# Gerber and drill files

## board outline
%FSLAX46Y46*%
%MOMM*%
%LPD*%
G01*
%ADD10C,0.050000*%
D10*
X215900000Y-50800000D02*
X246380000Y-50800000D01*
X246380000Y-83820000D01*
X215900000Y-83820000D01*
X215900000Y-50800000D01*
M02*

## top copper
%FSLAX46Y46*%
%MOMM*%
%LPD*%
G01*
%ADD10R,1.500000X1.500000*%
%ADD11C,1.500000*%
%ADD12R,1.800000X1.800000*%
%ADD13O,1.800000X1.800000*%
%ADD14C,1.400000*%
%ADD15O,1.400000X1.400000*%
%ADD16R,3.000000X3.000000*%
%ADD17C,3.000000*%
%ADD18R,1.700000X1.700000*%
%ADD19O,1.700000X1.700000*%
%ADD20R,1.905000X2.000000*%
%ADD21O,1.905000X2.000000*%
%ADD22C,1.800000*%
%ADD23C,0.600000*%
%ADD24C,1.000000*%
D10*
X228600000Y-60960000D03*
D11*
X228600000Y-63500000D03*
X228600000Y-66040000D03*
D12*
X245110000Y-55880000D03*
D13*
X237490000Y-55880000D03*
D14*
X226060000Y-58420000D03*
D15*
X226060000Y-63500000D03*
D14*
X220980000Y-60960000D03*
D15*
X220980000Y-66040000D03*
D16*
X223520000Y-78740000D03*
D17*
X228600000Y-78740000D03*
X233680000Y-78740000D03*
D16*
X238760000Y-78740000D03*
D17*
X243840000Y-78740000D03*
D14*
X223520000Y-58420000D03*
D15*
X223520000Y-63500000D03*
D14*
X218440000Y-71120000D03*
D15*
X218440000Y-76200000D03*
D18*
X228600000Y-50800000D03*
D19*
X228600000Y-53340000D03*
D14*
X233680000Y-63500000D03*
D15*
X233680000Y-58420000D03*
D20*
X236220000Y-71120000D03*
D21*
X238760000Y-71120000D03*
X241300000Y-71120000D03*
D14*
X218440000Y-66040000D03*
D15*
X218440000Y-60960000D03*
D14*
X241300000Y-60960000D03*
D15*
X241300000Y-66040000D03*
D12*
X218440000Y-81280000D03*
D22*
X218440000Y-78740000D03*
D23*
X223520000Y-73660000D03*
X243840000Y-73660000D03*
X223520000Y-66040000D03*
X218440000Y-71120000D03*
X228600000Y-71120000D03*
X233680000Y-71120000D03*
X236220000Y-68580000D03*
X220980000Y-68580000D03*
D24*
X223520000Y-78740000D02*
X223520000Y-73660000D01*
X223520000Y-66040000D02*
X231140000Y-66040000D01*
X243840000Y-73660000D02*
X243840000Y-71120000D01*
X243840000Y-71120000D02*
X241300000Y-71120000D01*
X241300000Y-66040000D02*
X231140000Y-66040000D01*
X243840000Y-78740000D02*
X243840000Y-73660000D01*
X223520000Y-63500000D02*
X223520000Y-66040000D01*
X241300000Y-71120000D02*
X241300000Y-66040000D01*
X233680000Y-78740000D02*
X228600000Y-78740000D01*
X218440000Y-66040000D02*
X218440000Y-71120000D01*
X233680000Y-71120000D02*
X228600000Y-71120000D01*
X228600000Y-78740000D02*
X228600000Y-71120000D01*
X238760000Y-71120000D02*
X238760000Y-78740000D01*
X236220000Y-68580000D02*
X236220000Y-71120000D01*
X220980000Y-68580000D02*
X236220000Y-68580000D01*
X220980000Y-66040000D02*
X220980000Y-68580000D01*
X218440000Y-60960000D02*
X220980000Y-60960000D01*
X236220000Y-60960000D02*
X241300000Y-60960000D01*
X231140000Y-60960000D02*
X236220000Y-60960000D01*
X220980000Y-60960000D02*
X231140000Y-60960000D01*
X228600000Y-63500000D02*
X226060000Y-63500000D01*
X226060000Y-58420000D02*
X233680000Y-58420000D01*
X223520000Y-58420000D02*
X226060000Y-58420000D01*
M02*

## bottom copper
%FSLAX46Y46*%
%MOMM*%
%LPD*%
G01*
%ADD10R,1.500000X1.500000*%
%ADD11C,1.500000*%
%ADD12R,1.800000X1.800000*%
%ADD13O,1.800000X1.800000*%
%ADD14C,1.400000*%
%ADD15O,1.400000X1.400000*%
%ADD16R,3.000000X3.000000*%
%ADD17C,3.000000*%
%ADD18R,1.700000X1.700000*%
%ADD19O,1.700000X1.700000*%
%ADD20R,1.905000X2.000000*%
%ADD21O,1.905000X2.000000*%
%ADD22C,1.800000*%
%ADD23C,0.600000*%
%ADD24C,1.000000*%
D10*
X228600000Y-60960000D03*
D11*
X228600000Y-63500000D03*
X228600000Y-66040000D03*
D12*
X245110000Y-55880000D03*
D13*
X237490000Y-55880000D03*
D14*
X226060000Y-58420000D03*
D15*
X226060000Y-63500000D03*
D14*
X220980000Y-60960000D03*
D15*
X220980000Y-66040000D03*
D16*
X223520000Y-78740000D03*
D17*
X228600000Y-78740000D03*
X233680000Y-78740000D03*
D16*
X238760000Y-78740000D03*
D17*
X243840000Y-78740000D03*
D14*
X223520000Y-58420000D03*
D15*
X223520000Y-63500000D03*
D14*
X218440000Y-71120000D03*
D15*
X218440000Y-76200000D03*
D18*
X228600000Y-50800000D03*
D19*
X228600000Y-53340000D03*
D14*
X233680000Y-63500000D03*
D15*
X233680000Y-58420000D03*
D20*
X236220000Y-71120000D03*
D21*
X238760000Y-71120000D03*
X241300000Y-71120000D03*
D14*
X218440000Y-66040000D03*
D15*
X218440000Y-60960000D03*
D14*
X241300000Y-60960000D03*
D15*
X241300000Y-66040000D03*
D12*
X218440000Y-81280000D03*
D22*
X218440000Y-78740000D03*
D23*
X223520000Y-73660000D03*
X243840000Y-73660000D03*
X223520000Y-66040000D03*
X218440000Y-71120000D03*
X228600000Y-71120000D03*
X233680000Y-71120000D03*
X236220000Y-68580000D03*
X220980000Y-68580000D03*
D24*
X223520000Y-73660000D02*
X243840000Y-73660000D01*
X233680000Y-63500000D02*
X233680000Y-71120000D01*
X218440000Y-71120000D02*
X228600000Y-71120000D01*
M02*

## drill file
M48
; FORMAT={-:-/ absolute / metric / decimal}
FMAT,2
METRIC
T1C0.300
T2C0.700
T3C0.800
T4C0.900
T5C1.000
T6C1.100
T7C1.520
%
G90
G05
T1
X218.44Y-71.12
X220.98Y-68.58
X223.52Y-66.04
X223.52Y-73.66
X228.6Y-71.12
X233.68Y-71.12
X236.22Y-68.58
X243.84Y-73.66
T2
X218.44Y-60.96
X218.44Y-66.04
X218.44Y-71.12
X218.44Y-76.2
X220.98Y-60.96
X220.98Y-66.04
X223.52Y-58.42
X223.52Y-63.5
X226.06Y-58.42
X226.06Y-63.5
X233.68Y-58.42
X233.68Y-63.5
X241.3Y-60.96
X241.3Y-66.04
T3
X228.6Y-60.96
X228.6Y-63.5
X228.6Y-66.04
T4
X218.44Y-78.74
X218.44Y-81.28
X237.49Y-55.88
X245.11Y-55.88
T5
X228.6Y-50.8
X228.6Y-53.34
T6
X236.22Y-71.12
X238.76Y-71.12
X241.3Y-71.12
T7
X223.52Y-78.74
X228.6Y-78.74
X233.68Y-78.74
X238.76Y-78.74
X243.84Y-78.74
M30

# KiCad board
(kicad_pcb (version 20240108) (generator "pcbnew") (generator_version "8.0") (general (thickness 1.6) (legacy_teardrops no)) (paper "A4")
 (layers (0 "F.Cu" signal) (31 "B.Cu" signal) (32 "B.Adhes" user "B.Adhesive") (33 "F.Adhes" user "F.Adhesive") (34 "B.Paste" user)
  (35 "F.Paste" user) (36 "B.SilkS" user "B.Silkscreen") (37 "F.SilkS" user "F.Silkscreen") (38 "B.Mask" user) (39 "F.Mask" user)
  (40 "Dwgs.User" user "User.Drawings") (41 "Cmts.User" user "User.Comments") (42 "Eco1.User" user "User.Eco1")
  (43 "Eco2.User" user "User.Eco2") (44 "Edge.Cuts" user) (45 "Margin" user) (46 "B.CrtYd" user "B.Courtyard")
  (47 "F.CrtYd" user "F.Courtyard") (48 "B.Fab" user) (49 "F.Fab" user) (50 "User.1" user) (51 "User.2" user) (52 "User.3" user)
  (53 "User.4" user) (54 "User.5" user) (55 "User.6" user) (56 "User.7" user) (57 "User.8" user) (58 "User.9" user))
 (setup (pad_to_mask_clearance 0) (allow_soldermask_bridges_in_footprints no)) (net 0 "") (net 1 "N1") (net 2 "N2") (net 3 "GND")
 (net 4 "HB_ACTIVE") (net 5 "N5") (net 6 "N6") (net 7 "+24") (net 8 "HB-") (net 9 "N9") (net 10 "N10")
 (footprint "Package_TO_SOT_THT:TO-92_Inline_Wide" (layer "F.Cu") (at 228.6 60.96 -90)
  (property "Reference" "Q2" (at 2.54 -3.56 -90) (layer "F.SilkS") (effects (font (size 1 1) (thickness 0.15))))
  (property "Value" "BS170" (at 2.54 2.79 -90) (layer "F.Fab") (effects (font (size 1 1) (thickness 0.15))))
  (pad "1" thru_hole rect (at 0 0 270) (size 1.5 1.5) (drill 0.8) (layers "*.Cu" "*.Mask") (remove_unused_layers no) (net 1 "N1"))
  (pad "2" thru_hole circle (at 2.54 0 270) (size 1.5 1.5) (drill 0.8) (layers "*.Cu" "*.Mask") (remove_unused_layers no) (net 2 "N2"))
  (pad "3" thru_hole circle (at 5.08 0 270) (size 1.5 1.5) (drill 0.8) (layers "*.Cu" "*.Mask") (remove_unused_layers no) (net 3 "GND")))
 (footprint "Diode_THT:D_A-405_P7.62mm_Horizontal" (layer "F.Cu") (at 245.11 55.88 180)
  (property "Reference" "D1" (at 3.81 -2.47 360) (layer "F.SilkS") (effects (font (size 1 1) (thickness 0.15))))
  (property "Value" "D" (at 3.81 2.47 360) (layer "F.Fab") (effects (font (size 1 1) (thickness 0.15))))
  (pad "1" thru_hole rect (at 0 0 180) (size 1.8 1.8) (drill 0.9) (layers "*.Cu" "*.Mask") (remove_unused_layers no) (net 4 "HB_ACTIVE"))
  (pad "2" thru_hole oval (at 7.62 0 180) (size 1.8 1.8) (drill 0.9) (layers "*.Cu" "*.Mask") (remove_unused_layers no) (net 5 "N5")))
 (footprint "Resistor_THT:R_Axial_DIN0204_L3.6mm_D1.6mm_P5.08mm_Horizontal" (layer "F.Cu") (at 226.06 58.42 -90)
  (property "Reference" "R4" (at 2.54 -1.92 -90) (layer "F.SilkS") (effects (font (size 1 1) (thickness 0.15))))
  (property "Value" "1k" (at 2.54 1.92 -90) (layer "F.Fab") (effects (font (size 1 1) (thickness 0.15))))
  (pad "1" thru_hole circle (at 0 0 270) (size 1.4 1.4) (drill 0.7) (layers "*.Cu" "*.Mask") (remove_unused_layers no) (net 5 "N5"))
  (pad "2" thru_hole oval (at 5.08 0 270) (size 1.4 1.4) (drill 0.7) (layers "*.Cu" "*.Mask") (remove_unused_layers no) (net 2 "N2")))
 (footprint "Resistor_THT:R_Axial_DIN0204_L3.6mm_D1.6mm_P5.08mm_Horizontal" (layer "F.Cu") (at 220.98 60.96 -90)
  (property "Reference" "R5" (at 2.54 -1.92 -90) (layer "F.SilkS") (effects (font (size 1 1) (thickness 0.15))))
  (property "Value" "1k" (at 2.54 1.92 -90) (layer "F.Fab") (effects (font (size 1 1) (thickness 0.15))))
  (pad "1" thru_hole circle (at 0 0 270) (size 1.4 1.4) (drill 0.7) (layers "*.Cu" "*.Mask") (remove_unused_layers no) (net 1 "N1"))
  (pad "2" thru_hole oval (at 5.08 0 270) (size 1.4 1.4) (drill 0.7) (layers "*.Cu" "*.Mask") (remove_unused_layers no) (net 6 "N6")))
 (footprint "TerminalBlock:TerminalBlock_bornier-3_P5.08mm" (layer "F.Cu") (at 223.52 78.74)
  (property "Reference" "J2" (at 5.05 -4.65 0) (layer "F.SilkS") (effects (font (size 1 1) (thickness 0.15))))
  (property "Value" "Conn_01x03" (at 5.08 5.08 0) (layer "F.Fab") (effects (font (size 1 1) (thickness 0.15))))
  (pad "1" thru_hole rect (at 0 0) (size 3 3) (drill 1.52) (layers "*.Cu" "*.Mask") (remove_unused_layers no) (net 3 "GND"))
  (pad "2" thru_hole circle (at 5.08 0) (size 3 3) (drill 1.52) (layers "*.Cu" "*.Mask") (remove_unused_layers no) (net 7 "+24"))
  (pad "3" thru_hole circle (at 10.16 0) (size 3 3) (drill 1.52) (layers "*.Cu" "*.Mask") (remove_unused_layers no) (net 7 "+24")))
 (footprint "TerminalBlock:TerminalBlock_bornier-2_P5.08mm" (layer "F.Cu") (at 238.76 78.74)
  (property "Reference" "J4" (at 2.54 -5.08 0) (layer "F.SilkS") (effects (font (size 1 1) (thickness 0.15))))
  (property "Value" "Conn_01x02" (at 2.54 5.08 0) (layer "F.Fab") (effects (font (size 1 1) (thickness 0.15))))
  (pad "1" thru_hole rect (at 0 0) (size 3 3) (drill 1.52) (layers "*.Cu" "*.Mask") (remove_unused_layers no) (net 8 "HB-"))
  (pad "2" thru_hole circle (at 5.08 0) (size 3 3) (drill 1.52) (layers "*.Cu" "*.Mask") (remove_unused_layers no) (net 3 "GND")))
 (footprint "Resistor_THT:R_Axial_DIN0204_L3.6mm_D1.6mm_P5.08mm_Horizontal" (layer "F.Cu") (at 223.52 58.42 -90)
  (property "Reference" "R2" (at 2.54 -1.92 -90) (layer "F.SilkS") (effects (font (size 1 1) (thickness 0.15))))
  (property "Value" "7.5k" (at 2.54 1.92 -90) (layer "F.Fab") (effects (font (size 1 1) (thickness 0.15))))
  (pad "1" thru_hole circle (at 0 0 270) (size 1.4 1.4) (drill 0.7) (layers "*.Cu" "*.Mask") (remove_unused_layers no) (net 5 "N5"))
  (pad "2" thru_hole oval (at 5.08 0 270) (size 1.4 1.4) (drill 0.7) (layers "*.Cu" "*.Mask") (remove_unused_layers no) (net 3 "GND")))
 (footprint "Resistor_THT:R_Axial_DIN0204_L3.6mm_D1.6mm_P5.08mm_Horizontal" (layer "F.Cu") (at 218.44 71.12 -90)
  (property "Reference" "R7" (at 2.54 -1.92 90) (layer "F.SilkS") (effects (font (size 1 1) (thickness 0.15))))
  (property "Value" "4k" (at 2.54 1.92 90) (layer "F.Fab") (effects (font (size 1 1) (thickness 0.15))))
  (pad "1" thru_hole circle (at 0 0 270) (size 1.4 1.4) (drill 0.7) (layers "*.Cu" "*.Mask") (remove_unused_layers no) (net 7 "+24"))
  (pad "2" thru_hole oval (at 5.08 0 270) (size 1.4 1.4) (drill 0.7) (layers "*.Cu" "*.Mask") (remove_unused_layers no) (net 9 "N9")))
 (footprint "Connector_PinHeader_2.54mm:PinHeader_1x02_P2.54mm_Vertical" (layer "F.Cu") (at 228.6 50.8)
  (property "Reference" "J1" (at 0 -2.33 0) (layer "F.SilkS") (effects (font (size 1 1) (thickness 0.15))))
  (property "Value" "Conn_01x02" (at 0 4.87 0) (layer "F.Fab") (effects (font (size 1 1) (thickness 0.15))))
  (pad "1" thru_hole rect (at 0 0) (size 1.7 1.7) (drill 1) (layers "*.Cu" "*.Mask") (remove_unused_layers no) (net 4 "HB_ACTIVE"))
  (pad "2" thru_hole oval (at 0 2.54) (size 1.7 1.7) (drill 1) (layers "*.Cu" "*.Mask") (remove_unused_layers no) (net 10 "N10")))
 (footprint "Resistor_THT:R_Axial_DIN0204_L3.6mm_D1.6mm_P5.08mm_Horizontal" (layer "F.Cu") (at 233.68 63.5 90)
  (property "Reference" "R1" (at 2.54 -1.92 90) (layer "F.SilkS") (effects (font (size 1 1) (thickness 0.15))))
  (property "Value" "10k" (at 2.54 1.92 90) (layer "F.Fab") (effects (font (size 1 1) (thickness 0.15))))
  (pad "1" thru_hole circle (at 0 0 90) (size 1.4 1.4) (drill 0.7) (layers "*.Cu" "*.Mask") (remove_unused_layers no) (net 7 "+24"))
  (pad "2" thru_hole oval (at 5.08 0 90) (size 1.4 1.4) (drill 0.7) (layers "*.Cu" "*.Mask") (remove_unused_layers no) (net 5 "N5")))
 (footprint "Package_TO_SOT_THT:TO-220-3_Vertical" (layer "F.Cu") (at 236.22 71.12)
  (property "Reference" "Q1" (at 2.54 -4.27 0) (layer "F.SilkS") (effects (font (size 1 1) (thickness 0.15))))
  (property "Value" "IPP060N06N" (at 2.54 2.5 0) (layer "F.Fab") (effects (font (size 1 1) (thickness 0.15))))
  (pad "1" thru_hole rect (at 0 0) (size 1.905 2) (drill 1.1) (layers "*.Cu" "*.Mask") (remove_unused_layers no) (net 6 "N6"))
  (pad "2" thru_hole oval (at 2.54 0) (size 1.905 2) (drill 1.1) (layers "*.Cu" "*.Mask") (remove_unused_layers no) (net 8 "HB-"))
  (pad "3" thru_hole oval (at 5.08 0) (size 1.905 2) (drill 1.1) (layers "*.Cu" "*.Mask") (remove_unused_layers no) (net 3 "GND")))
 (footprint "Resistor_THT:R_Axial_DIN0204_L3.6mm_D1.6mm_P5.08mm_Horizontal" (layer "F.Cu") (at 218.44 66.04 90)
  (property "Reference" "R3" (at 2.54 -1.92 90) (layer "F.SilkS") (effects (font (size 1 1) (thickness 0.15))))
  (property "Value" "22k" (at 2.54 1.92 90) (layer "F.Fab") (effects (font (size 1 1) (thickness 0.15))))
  (pad "1" thru_hole circle (at 0 0 90) (size 1.4 1.4) (drill 0.7) (layers "*.Cu" "*.Mask") (remove_unused_layers no) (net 7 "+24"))
  (pad "2" thru_hole oval (at 5.08 0 90) (size 1.4 1.4) (drill 0.7) (layers "*.Cu" "*.Mask") (remove_unused_layers no) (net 1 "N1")))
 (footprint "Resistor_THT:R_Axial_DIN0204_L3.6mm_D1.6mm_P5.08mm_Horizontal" (layer "F.Cu") (at 241.3 60.96 -90)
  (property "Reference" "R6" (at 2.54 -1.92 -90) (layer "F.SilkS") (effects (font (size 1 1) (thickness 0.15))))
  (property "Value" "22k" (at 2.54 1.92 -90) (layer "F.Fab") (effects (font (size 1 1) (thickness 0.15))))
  (pad "1" thru_hole circle (at 0 0 270) (size 1.4 1.4) (drill 0.7) (layers "*.Cu" "*.Mask") (remove_unused_layers no) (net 1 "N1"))
  (pad "2" thru_hole oval (at 5.08 0 270) (size 1.4 1.4) (drill 0.7) (layers "*.Cu" "*.Mask") (remove_unused_layers no) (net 3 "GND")))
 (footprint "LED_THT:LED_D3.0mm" (layer "F.Cu") (at 218.44 81.28 90)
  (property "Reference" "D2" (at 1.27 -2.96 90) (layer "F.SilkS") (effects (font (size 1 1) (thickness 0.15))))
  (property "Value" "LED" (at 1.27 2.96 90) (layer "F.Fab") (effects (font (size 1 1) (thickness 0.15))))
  (pad "1" thru_hole rect (at 0 0 90) (size 1.8 1.8) (drill 0.9) (layers "*.Cu" "*.Mask") (remove_unused_layers no) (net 8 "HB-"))
  (pad "2" thru_hole circle (at 2.54 0 90) (size 1.8 1.8) (drill 0.9) (layers "*.Cu" "*.Mask") (remove_unused_layers no) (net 9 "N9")))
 (gr_rect (start 215.9 50.8) (end 246.38 83.82) (stroke (width 0.05) (type default)) (fill none) (layer "Edge.Cuts"))
 (segment (start 223.52 78.74) (end 223.52 73.66) (width 1) (layer "F.Cu") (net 3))
 (segment (start 223.52 66.04) (end 231.14 66.04) (width 1) (layer "F.Cu") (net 3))
 (segment (start 243.84 73.66) (end 243.84 71.12) (width 1) (layer "F.Cu") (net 3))
 (segment (start 243.84 71.12) (end 241.3 71.12) (width 1) (layer "F.Cu") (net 3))
 (segment (start 241.3 66.04) (end 231.14 66.04) (width 1) (layer "F.Cu") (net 3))
 (segment (start 243.84 78.74) (end 243.84 73.66) (width 1) (layer "F.Cu") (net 3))
 (segment (start 223.52 63.5) (end 223.52 66.04) (width 1) (layer "F.Cu") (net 3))
 (segment (start 241.3 71.12) (end 241.3 66.04) (width 1) (layer "F.Cu") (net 3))
 (via (at 223.52 73.66) (size 0.6) (drill 0.3) (layers "F.Cu" "B.Cu") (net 3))
 (via (at 243.84 73.66) (size 0.6) (drill 0.3) (layers "F.Cu" "B.Cu") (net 3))
 (via (at 223.52 66.04) (size 0.6) (drill 0.3) (layers "F.Cu" "B.Cu") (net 3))
 (segment (start 223.52 73.66) (end 243.84 73.66) (width 1) (layer "B.Cu") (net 3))
 (segment (start 233.68 78.74) (end 228.6 78.74) (width 1) (layer "F.Cu") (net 7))
 (segment (start 218.44 66.04) (end 218.44 71.12) (width 1) (layer "F.Cu") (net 7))
 (segment (start 233.68 71.12) (end 228.6 71.12) (width 1) (layer "F.Cu") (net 7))
 (segment (start 228.6 78.74) (end 228.6 71.12) (width 1) (layer "F.Cu") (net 7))
 (via (at 218.44 71.12) (size 0.6) (drill 0.3) (layers "F.Cu" "B.Cu") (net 7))
 (via (at 228.6 71.12) (size 0.6) (drill 0.3) (layers "F.Cu" "B.Cu") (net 7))
 (via (at 233.68 71.12) (size 0.6) (drill 0.3) (layers "F.Cu" "B.Cu") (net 7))
 (segment (start 233.68 63.5) (end 233.68 71.12) (width 1) (layer "B.Cu") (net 7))
 (segment (start 218.44 71.12) (end 228.6 71.12) (width 1) (layer "B.Cu") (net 7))
 (segment (start 238.76 71.12) (end 238.76 78.74) (width 1) (layer "F.Cu") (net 8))
 (segment (start 236.22 68.58) (end 236.22 71.12) (width 1) (layer "F.Cu") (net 6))
 (segment (start 220.98 68.58) (end 236.22 68.58) (width 1) (layer "F.Cu") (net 6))
 (segment (start 220.98 66.04) (end 220.98 68.58) (width 1) (layer "F.Cu") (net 6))
 (via (at 236.22 68.58) (size 0.6) (drill 0.3) (layers "F.Cu" "B.Cu") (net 6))
 (via (at 220.98 68.58) (size 0.6) (drill 0.3) (layers "F.Cu" "B.Cu") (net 6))
 (segment (start 218.44 60.96) (end 220.98 60.96) (width 1) (layer "F.Cu") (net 1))
 (segment (start 236.22 60.96) (end 241.3 60.96) (width 1) (layer "F.Cu") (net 1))
 (segment (start 231.14 60.96) (end 236.22 60.96) (width 1) (layer "F.Cu") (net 1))
 (segment (start 220.98 60.96) (end 231.14 60.96) (width 1) (layer "F.Cu") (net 1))
 (segment (start 228.6 63.5) (end 226.06 63.5) (width 1) (layer "F.Cu") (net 2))
 (segment (start 226.06 58.42) (end 233.68 58.42) (width 1) (layer "F.Cu") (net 5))
 (segment (start 223.52 58.42) (end 226.06 58.42) (width 1) (layer "F.Cu") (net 5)))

